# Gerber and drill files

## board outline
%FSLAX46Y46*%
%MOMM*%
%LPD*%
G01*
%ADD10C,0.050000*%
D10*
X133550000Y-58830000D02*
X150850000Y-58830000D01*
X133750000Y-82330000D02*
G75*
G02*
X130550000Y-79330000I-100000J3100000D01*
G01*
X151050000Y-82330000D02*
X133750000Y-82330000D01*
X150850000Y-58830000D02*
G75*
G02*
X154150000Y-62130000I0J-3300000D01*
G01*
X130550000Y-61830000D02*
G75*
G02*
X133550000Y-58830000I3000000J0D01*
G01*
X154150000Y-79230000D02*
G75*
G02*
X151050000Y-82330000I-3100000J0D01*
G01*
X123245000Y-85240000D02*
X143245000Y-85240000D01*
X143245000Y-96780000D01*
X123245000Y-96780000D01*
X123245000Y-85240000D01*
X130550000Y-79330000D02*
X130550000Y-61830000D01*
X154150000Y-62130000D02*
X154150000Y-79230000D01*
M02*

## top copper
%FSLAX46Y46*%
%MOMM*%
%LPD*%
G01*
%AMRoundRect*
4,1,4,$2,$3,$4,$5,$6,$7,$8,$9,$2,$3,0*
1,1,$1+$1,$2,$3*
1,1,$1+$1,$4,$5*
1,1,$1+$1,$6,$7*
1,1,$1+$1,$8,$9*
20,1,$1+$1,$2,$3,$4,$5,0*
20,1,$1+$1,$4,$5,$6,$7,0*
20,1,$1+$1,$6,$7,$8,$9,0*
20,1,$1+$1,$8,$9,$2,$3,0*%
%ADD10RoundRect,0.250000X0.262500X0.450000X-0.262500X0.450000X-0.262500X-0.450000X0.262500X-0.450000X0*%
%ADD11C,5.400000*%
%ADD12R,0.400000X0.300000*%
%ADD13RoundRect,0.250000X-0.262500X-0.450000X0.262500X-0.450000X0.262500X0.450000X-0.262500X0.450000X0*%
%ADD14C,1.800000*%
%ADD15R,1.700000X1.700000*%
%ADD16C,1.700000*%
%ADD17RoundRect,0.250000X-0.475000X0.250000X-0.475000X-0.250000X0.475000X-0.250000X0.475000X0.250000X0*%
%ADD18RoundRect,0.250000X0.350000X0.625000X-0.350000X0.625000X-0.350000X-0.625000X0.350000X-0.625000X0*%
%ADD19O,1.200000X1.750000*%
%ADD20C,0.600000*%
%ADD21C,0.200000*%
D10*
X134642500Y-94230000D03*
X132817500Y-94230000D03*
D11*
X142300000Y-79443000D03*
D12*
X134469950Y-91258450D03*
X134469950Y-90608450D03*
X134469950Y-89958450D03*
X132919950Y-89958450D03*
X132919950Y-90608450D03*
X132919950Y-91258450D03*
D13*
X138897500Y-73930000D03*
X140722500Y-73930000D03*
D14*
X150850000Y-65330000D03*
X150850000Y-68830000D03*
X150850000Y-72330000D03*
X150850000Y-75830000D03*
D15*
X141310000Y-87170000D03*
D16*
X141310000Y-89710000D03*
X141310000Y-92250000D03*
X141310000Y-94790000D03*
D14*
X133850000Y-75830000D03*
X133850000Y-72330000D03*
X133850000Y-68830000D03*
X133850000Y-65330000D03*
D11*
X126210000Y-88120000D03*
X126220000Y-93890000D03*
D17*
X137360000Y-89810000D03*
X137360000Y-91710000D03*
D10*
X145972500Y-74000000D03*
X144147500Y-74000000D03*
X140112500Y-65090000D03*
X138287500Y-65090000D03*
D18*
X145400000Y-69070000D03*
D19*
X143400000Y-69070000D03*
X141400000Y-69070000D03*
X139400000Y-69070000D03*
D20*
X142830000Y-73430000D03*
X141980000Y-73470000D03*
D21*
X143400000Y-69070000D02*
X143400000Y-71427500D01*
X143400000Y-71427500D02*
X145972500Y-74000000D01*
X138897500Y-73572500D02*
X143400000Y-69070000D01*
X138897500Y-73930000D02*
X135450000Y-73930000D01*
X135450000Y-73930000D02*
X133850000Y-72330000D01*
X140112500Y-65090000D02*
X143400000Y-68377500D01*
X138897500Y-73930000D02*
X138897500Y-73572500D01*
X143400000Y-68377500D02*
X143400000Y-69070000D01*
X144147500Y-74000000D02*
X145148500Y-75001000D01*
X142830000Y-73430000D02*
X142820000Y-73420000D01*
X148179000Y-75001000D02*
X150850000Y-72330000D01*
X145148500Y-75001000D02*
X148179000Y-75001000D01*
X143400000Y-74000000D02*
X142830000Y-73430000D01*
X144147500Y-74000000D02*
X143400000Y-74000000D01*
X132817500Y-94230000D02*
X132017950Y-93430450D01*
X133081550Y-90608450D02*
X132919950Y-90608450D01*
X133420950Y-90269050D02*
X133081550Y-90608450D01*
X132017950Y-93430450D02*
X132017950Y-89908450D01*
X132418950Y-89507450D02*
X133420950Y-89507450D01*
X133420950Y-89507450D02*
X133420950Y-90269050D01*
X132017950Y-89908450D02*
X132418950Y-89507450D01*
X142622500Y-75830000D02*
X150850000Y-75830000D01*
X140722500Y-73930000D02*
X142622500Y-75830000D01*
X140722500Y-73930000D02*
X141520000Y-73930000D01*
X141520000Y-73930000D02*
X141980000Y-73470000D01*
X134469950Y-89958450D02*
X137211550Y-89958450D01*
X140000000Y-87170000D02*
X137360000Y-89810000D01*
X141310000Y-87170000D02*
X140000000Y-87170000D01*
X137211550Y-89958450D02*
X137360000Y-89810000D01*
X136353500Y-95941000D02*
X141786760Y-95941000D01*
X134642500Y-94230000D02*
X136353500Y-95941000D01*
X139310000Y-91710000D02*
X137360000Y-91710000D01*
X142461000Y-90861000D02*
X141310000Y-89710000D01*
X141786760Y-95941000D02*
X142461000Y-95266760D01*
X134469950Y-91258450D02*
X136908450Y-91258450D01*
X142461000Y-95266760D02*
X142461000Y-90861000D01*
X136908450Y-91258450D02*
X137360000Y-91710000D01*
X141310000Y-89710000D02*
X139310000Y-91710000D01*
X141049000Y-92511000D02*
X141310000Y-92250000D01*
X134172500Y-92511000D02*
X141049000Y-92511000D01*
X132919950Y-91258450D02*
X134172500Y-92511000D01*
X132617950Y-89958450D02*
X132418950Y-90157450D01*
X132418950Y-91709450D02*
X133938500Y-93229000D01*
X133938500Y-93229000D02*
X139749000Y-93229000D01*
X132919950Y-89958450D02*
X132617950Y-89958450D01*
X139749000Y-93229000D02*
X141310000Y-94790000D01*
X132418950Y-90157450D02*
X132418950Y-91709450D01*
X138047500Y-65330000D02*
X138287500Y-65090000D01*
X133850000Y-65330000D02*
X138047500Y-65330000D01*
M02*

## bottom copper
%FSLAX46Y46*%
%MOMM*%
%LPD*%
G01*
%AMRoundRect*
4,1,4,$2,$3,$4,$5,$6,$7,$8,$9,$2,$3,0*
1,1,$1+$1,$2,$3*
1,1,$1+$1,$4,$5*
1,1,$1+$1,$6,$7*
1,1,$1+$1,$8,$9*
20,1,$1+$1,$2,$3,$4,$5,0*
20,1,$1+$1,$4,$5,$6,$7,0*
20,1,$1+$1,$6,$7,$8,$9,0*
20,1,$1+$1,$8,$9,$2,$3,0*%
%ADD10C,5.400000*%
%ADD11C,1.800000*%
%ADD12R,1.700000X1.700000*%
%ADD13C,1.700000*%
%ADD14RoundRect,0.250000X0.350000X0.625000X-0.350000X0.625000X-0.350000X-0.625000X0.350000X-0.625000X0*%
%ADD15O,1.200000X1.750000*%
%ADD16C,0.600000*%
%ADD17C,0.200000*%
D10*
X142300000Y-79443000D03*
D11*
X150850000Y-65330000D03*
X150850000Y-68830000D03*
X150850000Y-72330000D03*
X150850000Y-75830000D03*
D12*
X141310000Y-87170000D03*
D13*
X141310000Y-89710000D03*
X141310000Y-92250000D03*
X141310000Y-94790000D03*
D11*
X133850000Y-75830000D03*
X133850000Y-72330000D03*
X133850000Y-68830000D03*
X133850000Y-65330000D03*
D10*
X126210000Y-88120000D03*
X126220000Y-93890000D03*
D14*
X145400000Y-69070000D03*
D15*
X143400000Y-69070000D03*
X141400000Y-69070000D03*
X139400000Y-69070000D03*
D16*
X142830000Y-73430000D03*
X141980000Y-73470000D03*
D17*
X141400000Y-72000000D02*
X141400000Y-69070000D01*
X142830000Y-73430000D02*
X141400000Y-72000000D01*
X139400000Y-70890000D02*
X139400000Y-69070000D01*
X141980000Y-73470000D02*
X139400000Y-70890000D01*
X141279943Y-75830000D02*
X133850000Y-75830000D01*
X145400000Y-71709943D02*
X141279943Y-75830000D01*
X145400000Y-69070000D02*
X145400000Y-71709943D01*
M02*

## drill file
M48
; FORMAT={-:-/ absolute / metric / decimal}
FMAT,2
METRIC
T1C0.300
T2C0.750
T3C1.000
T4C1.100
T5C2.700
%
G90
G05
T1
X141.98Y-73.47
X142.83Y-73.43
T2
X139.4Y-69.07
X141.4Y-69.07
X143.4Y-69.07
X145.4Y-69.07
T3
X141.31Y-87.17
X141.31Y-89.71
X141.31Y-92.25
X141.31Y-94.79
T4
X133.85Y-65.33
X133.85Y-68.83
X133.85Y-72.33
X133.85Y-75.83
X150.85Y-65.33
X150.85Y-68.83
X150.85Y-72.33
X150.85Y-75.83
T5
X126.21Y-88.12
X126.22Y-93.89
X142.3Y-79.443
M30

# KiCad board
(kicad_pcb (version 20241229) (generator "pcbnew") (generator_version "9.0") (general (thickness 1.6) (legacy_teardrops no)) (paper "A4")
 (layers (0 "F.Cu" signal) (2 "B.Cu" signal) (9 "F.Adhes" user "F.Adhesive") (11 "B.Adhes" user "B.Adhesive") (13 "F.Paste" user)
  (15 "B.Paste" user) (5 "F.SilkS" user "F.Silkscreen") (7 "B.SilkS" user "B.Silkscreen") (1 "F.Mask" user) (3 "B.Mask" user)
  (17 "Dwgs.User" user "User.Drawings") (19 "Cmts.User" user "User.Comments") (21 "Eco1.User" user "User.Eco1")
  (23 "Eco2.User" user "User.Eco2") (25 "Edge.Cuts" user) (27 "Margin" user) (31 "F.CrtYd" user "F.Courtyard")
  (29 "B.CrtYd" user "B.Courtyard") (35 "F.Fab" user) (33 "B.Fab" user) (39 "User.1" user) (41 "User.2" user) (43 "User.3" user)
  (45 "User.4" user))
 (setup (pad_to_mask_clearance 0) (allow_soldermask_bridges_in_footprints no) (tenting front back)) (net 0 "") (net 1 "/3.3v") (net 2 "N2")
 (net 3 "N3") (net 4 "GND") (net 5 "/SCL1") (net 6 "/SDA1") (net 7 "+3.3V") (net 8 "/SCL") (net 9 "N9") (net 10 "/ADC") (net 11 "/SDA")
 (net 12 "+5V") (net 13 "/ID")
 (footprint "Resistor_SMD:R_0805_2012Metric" (layer "F.Cu") (at 133.73 94.23 180)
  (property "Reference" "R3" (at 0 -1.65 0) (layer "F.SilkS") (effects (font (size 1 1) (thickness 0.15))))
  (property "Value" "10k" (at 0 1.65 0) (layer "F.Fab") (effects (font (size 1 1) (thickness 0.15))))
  (pad "1" smd roundrect (at -0.9125 0 180) (size 1.025 1.4) (layers "F.Cu" "F.Mask" "F.Paste") (roundrect_rratio 0.243902) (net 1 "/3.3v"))
  (pad "2" smd roundrect (at 0.9125 0 180) (size 1.025 1.4) (layers "F.Cu" "F.Mask" "F.Paste") (roundrect_rratio 0.243902) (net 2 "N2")))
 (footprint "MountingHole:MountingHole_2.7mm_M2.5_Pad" (layer "F.Cu") (at 142.3 79.443)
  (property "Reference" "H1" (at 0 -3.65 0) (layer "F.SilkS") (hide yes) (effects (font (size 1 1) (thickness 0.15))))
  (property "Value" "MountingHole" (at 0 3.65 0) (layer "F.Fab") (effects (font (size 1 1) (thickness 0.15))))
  (pad "1" thru_hole circle (at 0 0) (size 5.4 5.4) (drill 2.7) (layers "*.Cu" "*.Mask") (remove_unused_layers no) (zone_connect 2)))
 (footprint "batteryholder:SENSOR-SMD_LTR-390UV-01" (layer "F.Cu") (at 133.69495 90.60845 90)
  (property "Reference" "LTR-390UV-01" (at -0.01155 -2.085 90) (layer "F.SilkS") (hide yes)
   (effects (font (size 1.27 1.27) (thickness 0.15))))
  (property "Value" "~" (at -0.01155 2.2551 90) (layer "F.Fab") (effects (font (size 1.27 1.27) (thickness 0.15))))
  (pad "1" smd rect (at -0.65 0.775 90) (size 0.3 0.4) (layers "F.Cu" "F.Mask" "F.Paste") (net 1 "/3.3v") (solder_mask_margin 0.0508)
   (solder_paste_margin 0) (thermal_bridge_angle 0))
  (pad "2" smd rect (at 0 0.775 90) (size 0.3 0.4) (layers "F.Cu" "F.Mask" "F.Paste") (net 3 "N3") (solder_mask_margin 0.0508)
   (solder_paste_margin 0) (thermal_bridge_angle 0))
  (pad "3" smd rect (at 0.65 0.775 90) (size 0.3 0.4) (layers "F.Cu" "F.Mask" "F.Paste") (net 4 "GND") (solder_mask_margin 0.0508)
   (solder_paste_margin 0) (thermal_bridge_angle 0))
  (pad "4" smd rect (at 0.65 -0.775 90) (size 0.3 0.4) (layers "F.Cu" "F.Mask" "F.Paste") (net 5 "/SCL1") (solder_mask_margin 0.0508)
   (solder_paste_margin 0) (thermal_bridge_angle 0))
  (pad "5" smd rect (at 0 -0.775 90) (size 0.3 0.4) (layers "F.Cu" "F.Mask" "F.Paste") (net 2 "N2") (solder_mask_margin 0.0508)
   (solder_paste_margin 0) (thermal_bridge_angle 0))
  (pad "6" smd rect (at -0.65 -0.775 90) (size 0.3 0.4) (layers "F.Cu" "F.Mask" "F.Paste") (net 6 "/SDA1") (solder_mask_margin 0.0508)
   (solder_paste_margin 0) (thermal_bridge_angle 0))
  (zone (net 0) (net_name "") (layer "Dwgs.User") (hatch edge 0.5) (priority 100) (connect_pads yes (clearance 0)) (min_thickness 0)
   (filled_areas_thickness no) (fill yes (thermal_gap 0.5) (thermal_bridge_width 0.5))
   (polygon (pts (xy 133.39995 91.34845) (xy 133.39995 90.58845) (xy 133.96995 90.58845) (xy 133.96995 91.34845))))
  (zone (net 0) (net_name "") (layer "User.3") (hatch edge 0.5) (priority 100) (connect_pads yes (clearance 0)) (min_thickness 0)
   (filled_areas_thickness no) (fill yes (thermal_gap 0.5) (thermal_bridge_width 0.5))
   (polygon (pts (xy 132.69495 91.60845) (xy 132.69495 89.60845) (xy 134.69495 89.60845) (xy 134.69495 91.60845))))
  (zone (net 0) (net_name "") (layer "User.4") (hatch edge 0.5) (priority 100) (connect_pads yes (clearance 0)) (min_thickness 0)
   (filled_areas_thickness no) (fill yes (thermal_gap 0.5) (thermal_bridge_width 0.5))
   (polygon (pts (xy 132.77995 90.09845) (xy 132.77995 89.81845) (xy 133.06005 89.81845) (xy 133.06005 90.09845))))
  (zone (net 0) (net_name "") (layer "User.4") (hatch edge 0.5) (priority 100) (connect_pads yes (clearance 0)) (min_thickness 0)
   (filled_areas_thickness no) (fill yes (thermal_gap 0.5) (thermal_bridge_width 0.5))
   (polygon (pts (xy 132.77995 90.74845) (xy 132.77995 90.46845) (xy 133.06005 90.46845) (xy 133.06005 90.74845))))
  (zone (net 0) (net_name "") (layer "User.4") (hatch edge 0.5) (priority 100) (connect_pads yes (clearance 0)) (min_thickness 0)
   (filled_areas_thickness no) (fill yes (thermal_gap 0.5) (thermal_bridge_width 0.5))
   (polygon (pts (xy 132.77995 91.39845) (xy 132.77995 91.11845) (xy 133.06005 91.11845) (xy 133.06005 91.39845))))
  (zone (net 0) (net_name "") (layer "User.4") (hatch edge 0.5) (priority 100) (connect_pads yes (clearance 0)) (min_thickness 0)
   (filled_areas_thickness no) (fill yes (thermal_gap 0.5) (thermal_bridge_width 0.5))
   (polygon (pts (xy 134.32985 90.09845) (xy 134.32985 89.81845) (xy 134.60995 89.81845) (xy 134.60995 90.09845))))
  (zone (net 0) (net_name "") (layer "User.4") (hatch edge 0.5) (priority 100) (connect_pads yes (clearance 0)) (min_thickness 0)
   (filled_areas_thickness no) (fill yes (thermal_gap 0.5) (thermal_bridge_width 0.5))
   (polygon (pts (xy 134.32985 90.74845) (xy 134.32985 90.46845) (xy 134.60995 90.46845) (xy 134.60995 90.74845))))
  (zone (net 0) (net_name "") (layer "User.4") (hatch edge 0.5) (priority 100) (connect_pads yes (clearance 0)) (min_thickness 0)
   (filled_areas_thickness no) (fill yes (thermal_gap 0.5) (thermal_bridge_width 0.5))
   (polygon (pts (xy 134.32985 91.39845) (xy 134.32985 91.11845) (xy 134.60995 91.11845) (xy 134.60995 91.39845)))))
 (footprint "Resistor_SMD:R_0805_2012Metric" (layer "F.Cu") (at 139.81 73.93)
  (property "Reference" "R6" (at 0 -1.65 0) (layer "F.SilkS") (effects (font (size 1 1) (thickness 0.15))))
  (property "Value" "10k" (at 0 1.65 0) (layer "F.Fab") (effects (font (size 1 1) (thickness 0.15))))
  (pad "1" smd roundrect (at -0.9125 0) (size 1.025 1.4) (layers "F.Cu" "F.Mask" "F.Paste") (roundrect_rratio 0.243902) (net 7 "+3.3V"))
  (pad "2" smd roundrect (at 0.9125 0) (size 1.025 1.4) (layers "F.Cu" "F.Mask" "F.Paste") (roundrect_rratio 0.243902) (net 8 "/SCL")))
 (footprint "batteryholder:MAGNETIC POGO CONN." (layer "F.Cu") (at 150.85 70.58 -90)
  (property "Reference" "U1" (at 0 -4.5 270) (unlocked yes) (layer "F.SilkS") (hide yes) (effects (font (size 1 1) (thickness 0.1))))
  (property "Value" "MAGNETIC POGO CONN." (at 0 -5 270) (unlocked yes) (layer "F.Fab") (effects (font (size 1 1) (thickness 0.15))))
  (pad "1" thru_hole circle (at -5.25 0 270) (size 1.8 1.8) (drill 1.1) (layers "*.Cu" "*.Mask") (remove_unused_layers no) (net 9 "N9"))
  (pad "2" thru_hole circle (at -1.75 0 270) (size 1.8 1.8) (drill 1.1) (layers "*.Cu" "*.Mask") (remove_unused_layers no) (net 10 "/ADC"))
  (pad "3" thru_hole circle (at 1.75 0 270) (size 1.8 1.8) (drill 1.1) (layers "*.Cu" "*.Mask") (remove_unused_layers no) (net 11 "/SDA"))
  (pad "4" thru_hole circle (at 5.25 0 270) (size 1.8 1.8) (drill 1.1) (layers "*.Cu" "*.Mask") (remove_unused_layers no) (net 8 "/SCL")))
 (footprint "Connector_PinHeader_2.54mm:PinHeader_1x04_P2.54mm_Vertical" (layer "F.Cu") (at 141.31 87.17)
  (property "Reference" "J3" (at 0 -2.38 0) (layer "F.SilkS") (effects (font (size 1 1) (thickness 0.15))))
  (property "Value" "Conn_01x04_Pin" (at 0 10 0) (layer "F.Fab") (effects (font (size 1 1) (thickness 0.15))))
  (pad "1" thru_hole rect (at 0 0) (size 1.7 1.7) (drill 1) (layers "*.Cu" "*.Mask") (remove_unused_layers no) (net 4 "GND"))
  (pad "2" thru_hole circle (at 0 2.54) (size 1.7 1.7) (drill 1) (layers "*.Cu" "*.Mask") (remove_unused_layers no) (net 1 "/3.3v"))
  (pad "3" thru_hole circle (at 0 5.08) (size 1.7 1.7) (drill 1) (layers "*.Cu" "*.Mask") (remove_unused_layers no) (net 6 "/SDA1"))
  (pad "4" thru_hole circle (at 0 7.62) (size 1.7 1.7) (drill 1) (layers "*.Cu" "*.Mask") (remove_unused_layers no) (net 5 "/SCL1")))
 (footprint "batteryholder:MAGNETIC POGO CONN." (layer "F.Cu") (at 133.85 70.58 90)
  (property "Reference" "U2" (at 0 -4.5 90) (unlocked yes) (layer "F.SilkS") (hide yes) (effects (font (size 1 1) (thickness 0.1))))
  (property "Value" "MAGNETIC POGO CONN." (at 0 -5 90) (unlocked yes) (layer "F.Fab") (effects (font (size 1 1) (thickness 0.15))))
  (pad "1" thru_hole circle (at -5.25 0 90) (size 1.8 1.8) (drill 1.1) (layers "*.Cu" "*.Mask") (remove_unused_layers no) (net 4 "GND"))
  (pad "2" thru_hole circle (at -1.75 0 90) (size 1.8 1.8) (drill 1.1) (layers "*.Cu" "*.Mask") (remove_unused_layers no) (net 7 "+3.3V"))
  (pad "3" thru_hole circle (at 1.75 0 90) (size 1.8 1.8) (drill 1.1) (layers "*.Cu" "*.Mask") (remove_unused_layers no) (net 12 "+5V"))
  (pad "4" thru_hole circle (at 5.25 0 90) (size 1.8 1.8) (drill 1.1) (layers "*.Cu" "*.Mask") (remove_unused_layers no) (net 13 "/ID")))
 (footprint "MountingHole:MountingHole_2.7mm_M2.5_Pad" (layer "F.Cu") (at 126.21 88.12)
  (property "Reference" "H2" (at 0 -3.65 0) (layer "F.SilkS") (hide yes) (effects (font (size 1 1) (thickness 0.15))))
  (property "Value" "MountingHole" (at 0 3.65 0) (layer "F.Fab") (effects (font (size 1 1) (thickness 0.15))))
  (pad "1" thru_hole circle (at 0 0) (size 5.4 5.4) (drill 2.7) (layers "*.Cu" "*.Mask") (remove_unused_layers no) (zone_connect 2)))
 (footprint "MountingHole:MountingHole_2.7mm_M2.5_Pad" (layer "F.Cu") (at 126.22 93.89)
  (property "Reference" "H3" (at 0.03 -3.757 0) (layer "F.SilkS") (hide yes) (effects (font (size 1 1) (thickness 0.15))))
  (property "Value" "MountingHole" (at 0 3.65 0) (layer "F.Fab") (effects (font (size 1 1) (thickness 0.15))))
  (pad "1" thru_hole circle (at 0 0) (size 5.4 5.4) (drill 2.7) (layers "*.Cu" "*.Mask") (remove_unused_layers no) (zone_connect 2)))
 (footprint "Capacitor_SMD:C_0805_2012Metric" (layer "F.Cu") (at 137.36 90.76 -90)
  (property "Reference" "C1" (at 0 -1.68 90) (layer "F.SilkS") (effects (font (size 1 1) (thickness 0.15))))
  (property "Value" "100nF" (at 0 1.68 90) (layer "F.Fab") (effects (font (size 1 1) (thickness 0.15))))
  (pad "1" smd roundrect (at -0.95 0 270) (size 1 1.45) (layers "F.Cu" "F.Mask" "F.Paste") (roundrect_rratio 0.25) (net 4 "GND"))
  (pad "2" smd roundrect (at 0.95 0 270) (size 1 1.45) (layers "F.Cu" "F.Mask" "F.Paste") (roundrect_rratio 0.25) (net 1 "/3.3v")))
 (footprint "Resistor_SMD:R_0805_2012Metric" (layer "F.Cu") (at 145.06 74 180)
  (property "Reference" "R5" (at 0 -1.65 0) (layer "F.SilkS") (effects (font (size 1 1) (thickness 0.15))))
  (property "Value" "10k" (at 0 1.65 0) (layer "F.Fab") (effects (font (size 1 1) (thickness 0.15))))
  (pad "1" smd roundrect (at -0.9125 0 180) (size 1.025 1.4) (layers "F.Cu" "F.Mask" "F.Paste") (roundrect_rratio 0.243902) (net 7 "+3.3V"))
  (pad "2" smd roundrect (at 0.9125 0 180) (size 1.025 1.4) (layers "F.Cu" "F.Mask" "F.Paste") (roundrect_rratio 0.243902) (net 11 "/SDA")))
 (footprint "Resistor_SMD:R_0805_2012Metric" (layer "F.Cu") (at 139.2 65.09 180)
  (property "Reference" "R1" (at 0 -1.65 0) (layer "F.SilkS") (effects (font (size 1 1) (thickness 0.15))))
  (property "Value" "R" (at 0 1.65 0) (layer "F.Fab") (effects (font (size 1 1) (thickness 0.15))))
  (pad "1" smd roundrect (at -0.9125 0 180) (size 1.025 1.4) (layers "F.Cu" "F.Mask" "F.Paste") (roundrect_rratio 0.243902) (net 7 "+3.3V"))
  (pad "2" smd roundrect (at 0.9125 0 180) (size 1.025 1.4) (layers "F.Cu" "F.Mask" "F.Paste") (roundrect_rratio 0.243902) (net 13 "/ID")))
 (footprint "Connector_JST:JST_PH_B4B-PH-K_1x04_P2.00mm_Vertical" (layer "B.Cu") (at 145.4 69.07 180)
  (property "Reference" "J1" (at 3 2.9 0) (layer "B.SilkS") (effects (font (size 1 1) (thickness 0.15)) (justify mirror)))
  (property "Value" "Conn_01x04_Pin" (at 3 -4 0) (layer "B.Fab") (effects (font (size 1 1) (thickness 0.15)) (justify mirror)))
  (pad "1" thru_hole roundrect (at 0 0 180) (size 1.2 1.75) (drill 0.75) (layers "*.Cu" "*.Mask") (remove_unused_layers no)
   (roundrect_rratio 0.208333) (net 4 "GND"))
  (pad "2" thru_hole oval (at 2 0 180) (size 1.2 1.75) (drill 0.75) (layers "*.Cu" "*.Mask") (remove_unused_layers no) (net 7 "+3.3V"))
  (pad "3" thru_hole oval (at 4 0 180) (size 1.2 1.75) (drill 0.75) (layers "*.Cu" "*.Mask") (remove_unused_layers no) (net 11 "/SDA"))
  (pad "4" thru_hole oval (at 6 0 180) (size 1.2 1.75) (drill 0.75) (layers "*.Cu" "*.Mask") (remove_unused_layers no) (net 8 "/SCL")))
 (gr_line (start 133.55 58.83) (end 150.85 58.83) (stroke (width 0.05) (type default)) (layer "Edge.Cuts"))
 (gr_arc (start 133.75 82.33) (mid 131.52868 81.492742) (end 130.55 79.33) (stroke (width 0.05) (type default)) (layer "Edge.Cuts"))
 (gr_line (start 151.05 82.33) (end 133.75 82.33) (stroke (width 0.05) (type default)) (layer "Edge.Cuts"))
 (gr_arc (start 150.85 58.83) (mid 153.183452 59.796548) (end 154.15 62.13) (stroke (width 0.05) (type default)) (layer "Edge.Cuts"))
 (gr_arc (start 130.55 61.83) (mid 131.42868 59.70868) (end 133.55 58.83) (stroke (width 0.05) (type default)) (layer "Edge.Cuts"))
 (gr_arc (start 154.15 79.23) (mid 153.242031 81.422031) (end 151.05 82.33) (stroke (width 0.05) (type default)) (layer "Edge.Cuts"))
 (gr_rect (start 123.245 85.24) (end 143.245 96.78) (stroke (width 0.05) (type solid)) (fill no) (layer "Edge.Cuts"))
 (gr_line (start 130.55 79.33) (end 130.55 61.83) (stroke (width 0.05) (type default)) (layer "Edge.Cuts"))
 (gr_line (start 154.15 62.13) (end 154.15 79.23) (stroke (width 0.05) (type default)) (layer "Edge.Cuts"))
 (segment (start 143.4 69.07) (end 143.4 71.4275) (width 0.2) (layer "F.Cu") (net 7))
 (segment (start 143.4 71.4275) (end 145.9725 74) (width 0.2) (layer "F.Cu") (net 7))
 (segment (start 138.8975 73.5725) (end 143.4 69.07) (width 0.2) (layer "F.Cu") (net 7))
 (segment (start 138.8975 73.93) (end 135.45 73.93) (width 0.2) (layer "F.Cu") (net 7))
 (segment (start 135.45 73.93) (end 133.85 72.33) (width 0.2) (layer "F.Cu") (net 7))
 (segment (start 140.1125 65.09) (end 143.4 68.3775) (width 0.2) (layer "F.Cu") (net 7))
 (segment (start 138.8975 73.93) (end 138.8975 73.5725) (width 0.2) (layer "F.Cu") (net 7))
 (segment (start 143.4 68.3775) (end 143.4 69.07) (width 0.2) (layer "F.Cu") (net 7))
 (segment (start 144.1475 74) (end 145.1485 75.001) (width 0.2) (layer "F.Cu") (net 11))
 (segment (start 142.83 73.43) (end 142.82 73.42) (width 0.2) (layer "F.Cu") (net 11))
 (segment (start 148.179 75.001) (end 150.85 72.33) (width 0.2) (layer "F.Cu") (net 11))
 (segment (start 145.1485 75.001) (end 148.179 75.001) (width 0.2) (layer "F.Cu") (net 11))
 (segment (start 143.4 74) (end 142.83 73.43) (width 0.2) (layer "F.Cu") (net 11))
 (segment (start 144.1475 74) (end 143.4 74) (width 0.2) (layer "F.Cu") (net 11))
 (via blind (at 142.83 73.43) (size 0.6) (drill 0.3) (layers "F.Cu" "B.Cu") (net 11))
 (segment (start 141.4 72) (end 141.4 69.07) (width 0.2) (layer "B.Cu") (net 11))
 (segment (start 142.83 73.43) (end 141.4 72) (width 0.2) (layer "B.Cu") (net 11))
 (segment (start 132.8175 94.23) (end 132.01795 93.43045) (width 0.2) (layer "F.Cu") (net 2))
 (segment (start 133.08155 90.60845) (end 132.91995 90.60845) (width 0.2) (layer "F.Cu") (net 2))
 (segment (start 133.42095 90.26905) (end 133.08155 90.60845) (width 0.2) (layer "F.Cu") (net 2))
 (segment (start 132.01795 93.43045) (end 132.01795 89.90845) (width 0.2) (layer "F.Cu") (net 2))
 (segment (start 132.41895 89.50745) (end 133.42095 89.50745) (width 0.2) (layer "F.Cu") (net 2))
 (segment (start 133.42095 89.50745) (end 133.42095 90.26905) (width 0.2) (layer "F.Cu") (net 2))
 (segment (start 132.01795 89.90845) (end 132.41895 89.50745) (width 0.2) (layer "F.Cu") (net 2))
 (segment (start 142.6225 75.83) (end 150.85 75.83) (width 0.2) (layer "F.Cu") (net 8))
 (segment (start 140.7225 73.93) (end 142.6225 75.83) (width 0.2) (layer "F.Cu") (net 8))
 (segment (start 140.7225 73.93) (end 141.52 73.93) (width 0.2) (layer "F.Cu") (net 8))
 (segment (start 141.52 73.93) (end 141.98 73.47) (width 0.2) (layer "F.Cu") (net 8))
 (via blind (at 141.98 73.47) (size 0.6) (drill 0.3) (layers "F.Cu" "B.Cu") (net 8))
 (segment (start 139.4 70.89) (end 139.4 69.07) (width 0.2) (layer "B.Cu") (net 8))
 (segment (start 141.98 73.47) (end 139.4 70.89) (width 0.2) (layer "B.Cu") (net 8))
 (segment (start 134.46995 89.95845) (end 137.21155 89.95845) (width 0.2) (layer "F.Cu") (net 4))
 (segment (start 140 87.17) (end 137.36 89.81) (width 0.2) (layer "F.Cu") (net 4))
 (segment (start 141.31 87.17) (end 140 87.17) (width 0.2) (layer "F.Cu") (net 4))
 (segment (start 137.21155 89.95845) (end 137.36 89.81) (width 0.2) (layer "F.Cu") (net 4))
 (segment (start 141.279943 75.83) (end 133.85 75.83) (width 0.2) (layer "B.Cu") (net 4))
 (segment (start 145.4 71.709943) (end 141.279943 75.83) (width 0.2) (layer "B.Cu") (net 4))
 (segment (start 145.4 69.07) (end 145.4 71.709943) (width 0.2) (layer "B.Cu") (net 4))
 (segment (start 136.3535 95.941) (end 141.78676 95.941) (width 0.2) (layer "F.Cu") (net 1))
 (segment (start 134.6425 94.23) (end 136.3535 95.941) (width 0.2) (layer "F.Cu") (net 1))
 (segment (start 139.31 91.71) (end 137.36 91.71) (width 0.2) (layer "F.Cu") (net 1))
 (segment (start 142.461 90.861) (end 141.31 89.71) (width 0.2) (layer "F.Cu") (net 1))
 (segment (start 141.78676 95.941) (end 142.461 95.26676) (width 0.2) (layer "F.Cu") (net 1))
 (segment (start 134.46995 91.25845) (end 136.90845 91.25845) (width 0.2) (layer "F.Cu") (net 1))
 (segment (start 142.461 95.26676) (end 142.461 90.861) (width 0.2) (layer "F.Cu") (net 1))
 (segment (start 136.90845 91.25845) (end 137.36 91.71) (width 0.2) (layer "F.Cu") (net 1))
 (segment (start 141.31 89.71) (end 139.31 91.71) (width 0.2) (layer "F.Cu") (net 1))
 (segment (start 141.049 92.511) (end 141.31 92.25) (width 0.2) (layer "F.Cu") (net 6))
 (segment (start 134.1725 92.511) (end 141.049 92.511) (width 0.2) (layer "F.Cu") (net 6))
 (segment (start 132.91995 91.25845) (end 134.1725 92.511) (width 0.2) (layer "F.Cu") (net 6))
 (segment (start 132.61795 89.95845) (end 132.41895 90.15745) (width 0.2) (layer "F.Cu") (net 5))
 (segment (start 132.41895 91.70945) (end 133.9385 93.229) (width 0.2) (layer "F.Cu") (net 5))
 (segment (start 133.9385 93.229) (end 139.749 93.229) (width 0.2) (layer "F.Cu") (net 5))
 (segment (start 132.91995 89.95845) (end 132.61795 89.95845) (width 0.2) (layer "F.Cu") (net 5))
 (segment (start 139.749 93.229) (end 141.31 94.79) (width 0.2) (layer "F.Cu") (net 5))
 (segment (start 132.41895 90.15745) (end 132.41895 91.70945) (width 0.2) (layer "F.Cu") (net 5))
 (segment (start 138.0475 65.33) (end 138.2875 65.09) (width 0.2) (layer "F.Cu") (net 13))
 (segment (start 133.85 65.33) (end 138.0475 65.33) (width 0.2) (layer "F.Cu") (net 13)))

